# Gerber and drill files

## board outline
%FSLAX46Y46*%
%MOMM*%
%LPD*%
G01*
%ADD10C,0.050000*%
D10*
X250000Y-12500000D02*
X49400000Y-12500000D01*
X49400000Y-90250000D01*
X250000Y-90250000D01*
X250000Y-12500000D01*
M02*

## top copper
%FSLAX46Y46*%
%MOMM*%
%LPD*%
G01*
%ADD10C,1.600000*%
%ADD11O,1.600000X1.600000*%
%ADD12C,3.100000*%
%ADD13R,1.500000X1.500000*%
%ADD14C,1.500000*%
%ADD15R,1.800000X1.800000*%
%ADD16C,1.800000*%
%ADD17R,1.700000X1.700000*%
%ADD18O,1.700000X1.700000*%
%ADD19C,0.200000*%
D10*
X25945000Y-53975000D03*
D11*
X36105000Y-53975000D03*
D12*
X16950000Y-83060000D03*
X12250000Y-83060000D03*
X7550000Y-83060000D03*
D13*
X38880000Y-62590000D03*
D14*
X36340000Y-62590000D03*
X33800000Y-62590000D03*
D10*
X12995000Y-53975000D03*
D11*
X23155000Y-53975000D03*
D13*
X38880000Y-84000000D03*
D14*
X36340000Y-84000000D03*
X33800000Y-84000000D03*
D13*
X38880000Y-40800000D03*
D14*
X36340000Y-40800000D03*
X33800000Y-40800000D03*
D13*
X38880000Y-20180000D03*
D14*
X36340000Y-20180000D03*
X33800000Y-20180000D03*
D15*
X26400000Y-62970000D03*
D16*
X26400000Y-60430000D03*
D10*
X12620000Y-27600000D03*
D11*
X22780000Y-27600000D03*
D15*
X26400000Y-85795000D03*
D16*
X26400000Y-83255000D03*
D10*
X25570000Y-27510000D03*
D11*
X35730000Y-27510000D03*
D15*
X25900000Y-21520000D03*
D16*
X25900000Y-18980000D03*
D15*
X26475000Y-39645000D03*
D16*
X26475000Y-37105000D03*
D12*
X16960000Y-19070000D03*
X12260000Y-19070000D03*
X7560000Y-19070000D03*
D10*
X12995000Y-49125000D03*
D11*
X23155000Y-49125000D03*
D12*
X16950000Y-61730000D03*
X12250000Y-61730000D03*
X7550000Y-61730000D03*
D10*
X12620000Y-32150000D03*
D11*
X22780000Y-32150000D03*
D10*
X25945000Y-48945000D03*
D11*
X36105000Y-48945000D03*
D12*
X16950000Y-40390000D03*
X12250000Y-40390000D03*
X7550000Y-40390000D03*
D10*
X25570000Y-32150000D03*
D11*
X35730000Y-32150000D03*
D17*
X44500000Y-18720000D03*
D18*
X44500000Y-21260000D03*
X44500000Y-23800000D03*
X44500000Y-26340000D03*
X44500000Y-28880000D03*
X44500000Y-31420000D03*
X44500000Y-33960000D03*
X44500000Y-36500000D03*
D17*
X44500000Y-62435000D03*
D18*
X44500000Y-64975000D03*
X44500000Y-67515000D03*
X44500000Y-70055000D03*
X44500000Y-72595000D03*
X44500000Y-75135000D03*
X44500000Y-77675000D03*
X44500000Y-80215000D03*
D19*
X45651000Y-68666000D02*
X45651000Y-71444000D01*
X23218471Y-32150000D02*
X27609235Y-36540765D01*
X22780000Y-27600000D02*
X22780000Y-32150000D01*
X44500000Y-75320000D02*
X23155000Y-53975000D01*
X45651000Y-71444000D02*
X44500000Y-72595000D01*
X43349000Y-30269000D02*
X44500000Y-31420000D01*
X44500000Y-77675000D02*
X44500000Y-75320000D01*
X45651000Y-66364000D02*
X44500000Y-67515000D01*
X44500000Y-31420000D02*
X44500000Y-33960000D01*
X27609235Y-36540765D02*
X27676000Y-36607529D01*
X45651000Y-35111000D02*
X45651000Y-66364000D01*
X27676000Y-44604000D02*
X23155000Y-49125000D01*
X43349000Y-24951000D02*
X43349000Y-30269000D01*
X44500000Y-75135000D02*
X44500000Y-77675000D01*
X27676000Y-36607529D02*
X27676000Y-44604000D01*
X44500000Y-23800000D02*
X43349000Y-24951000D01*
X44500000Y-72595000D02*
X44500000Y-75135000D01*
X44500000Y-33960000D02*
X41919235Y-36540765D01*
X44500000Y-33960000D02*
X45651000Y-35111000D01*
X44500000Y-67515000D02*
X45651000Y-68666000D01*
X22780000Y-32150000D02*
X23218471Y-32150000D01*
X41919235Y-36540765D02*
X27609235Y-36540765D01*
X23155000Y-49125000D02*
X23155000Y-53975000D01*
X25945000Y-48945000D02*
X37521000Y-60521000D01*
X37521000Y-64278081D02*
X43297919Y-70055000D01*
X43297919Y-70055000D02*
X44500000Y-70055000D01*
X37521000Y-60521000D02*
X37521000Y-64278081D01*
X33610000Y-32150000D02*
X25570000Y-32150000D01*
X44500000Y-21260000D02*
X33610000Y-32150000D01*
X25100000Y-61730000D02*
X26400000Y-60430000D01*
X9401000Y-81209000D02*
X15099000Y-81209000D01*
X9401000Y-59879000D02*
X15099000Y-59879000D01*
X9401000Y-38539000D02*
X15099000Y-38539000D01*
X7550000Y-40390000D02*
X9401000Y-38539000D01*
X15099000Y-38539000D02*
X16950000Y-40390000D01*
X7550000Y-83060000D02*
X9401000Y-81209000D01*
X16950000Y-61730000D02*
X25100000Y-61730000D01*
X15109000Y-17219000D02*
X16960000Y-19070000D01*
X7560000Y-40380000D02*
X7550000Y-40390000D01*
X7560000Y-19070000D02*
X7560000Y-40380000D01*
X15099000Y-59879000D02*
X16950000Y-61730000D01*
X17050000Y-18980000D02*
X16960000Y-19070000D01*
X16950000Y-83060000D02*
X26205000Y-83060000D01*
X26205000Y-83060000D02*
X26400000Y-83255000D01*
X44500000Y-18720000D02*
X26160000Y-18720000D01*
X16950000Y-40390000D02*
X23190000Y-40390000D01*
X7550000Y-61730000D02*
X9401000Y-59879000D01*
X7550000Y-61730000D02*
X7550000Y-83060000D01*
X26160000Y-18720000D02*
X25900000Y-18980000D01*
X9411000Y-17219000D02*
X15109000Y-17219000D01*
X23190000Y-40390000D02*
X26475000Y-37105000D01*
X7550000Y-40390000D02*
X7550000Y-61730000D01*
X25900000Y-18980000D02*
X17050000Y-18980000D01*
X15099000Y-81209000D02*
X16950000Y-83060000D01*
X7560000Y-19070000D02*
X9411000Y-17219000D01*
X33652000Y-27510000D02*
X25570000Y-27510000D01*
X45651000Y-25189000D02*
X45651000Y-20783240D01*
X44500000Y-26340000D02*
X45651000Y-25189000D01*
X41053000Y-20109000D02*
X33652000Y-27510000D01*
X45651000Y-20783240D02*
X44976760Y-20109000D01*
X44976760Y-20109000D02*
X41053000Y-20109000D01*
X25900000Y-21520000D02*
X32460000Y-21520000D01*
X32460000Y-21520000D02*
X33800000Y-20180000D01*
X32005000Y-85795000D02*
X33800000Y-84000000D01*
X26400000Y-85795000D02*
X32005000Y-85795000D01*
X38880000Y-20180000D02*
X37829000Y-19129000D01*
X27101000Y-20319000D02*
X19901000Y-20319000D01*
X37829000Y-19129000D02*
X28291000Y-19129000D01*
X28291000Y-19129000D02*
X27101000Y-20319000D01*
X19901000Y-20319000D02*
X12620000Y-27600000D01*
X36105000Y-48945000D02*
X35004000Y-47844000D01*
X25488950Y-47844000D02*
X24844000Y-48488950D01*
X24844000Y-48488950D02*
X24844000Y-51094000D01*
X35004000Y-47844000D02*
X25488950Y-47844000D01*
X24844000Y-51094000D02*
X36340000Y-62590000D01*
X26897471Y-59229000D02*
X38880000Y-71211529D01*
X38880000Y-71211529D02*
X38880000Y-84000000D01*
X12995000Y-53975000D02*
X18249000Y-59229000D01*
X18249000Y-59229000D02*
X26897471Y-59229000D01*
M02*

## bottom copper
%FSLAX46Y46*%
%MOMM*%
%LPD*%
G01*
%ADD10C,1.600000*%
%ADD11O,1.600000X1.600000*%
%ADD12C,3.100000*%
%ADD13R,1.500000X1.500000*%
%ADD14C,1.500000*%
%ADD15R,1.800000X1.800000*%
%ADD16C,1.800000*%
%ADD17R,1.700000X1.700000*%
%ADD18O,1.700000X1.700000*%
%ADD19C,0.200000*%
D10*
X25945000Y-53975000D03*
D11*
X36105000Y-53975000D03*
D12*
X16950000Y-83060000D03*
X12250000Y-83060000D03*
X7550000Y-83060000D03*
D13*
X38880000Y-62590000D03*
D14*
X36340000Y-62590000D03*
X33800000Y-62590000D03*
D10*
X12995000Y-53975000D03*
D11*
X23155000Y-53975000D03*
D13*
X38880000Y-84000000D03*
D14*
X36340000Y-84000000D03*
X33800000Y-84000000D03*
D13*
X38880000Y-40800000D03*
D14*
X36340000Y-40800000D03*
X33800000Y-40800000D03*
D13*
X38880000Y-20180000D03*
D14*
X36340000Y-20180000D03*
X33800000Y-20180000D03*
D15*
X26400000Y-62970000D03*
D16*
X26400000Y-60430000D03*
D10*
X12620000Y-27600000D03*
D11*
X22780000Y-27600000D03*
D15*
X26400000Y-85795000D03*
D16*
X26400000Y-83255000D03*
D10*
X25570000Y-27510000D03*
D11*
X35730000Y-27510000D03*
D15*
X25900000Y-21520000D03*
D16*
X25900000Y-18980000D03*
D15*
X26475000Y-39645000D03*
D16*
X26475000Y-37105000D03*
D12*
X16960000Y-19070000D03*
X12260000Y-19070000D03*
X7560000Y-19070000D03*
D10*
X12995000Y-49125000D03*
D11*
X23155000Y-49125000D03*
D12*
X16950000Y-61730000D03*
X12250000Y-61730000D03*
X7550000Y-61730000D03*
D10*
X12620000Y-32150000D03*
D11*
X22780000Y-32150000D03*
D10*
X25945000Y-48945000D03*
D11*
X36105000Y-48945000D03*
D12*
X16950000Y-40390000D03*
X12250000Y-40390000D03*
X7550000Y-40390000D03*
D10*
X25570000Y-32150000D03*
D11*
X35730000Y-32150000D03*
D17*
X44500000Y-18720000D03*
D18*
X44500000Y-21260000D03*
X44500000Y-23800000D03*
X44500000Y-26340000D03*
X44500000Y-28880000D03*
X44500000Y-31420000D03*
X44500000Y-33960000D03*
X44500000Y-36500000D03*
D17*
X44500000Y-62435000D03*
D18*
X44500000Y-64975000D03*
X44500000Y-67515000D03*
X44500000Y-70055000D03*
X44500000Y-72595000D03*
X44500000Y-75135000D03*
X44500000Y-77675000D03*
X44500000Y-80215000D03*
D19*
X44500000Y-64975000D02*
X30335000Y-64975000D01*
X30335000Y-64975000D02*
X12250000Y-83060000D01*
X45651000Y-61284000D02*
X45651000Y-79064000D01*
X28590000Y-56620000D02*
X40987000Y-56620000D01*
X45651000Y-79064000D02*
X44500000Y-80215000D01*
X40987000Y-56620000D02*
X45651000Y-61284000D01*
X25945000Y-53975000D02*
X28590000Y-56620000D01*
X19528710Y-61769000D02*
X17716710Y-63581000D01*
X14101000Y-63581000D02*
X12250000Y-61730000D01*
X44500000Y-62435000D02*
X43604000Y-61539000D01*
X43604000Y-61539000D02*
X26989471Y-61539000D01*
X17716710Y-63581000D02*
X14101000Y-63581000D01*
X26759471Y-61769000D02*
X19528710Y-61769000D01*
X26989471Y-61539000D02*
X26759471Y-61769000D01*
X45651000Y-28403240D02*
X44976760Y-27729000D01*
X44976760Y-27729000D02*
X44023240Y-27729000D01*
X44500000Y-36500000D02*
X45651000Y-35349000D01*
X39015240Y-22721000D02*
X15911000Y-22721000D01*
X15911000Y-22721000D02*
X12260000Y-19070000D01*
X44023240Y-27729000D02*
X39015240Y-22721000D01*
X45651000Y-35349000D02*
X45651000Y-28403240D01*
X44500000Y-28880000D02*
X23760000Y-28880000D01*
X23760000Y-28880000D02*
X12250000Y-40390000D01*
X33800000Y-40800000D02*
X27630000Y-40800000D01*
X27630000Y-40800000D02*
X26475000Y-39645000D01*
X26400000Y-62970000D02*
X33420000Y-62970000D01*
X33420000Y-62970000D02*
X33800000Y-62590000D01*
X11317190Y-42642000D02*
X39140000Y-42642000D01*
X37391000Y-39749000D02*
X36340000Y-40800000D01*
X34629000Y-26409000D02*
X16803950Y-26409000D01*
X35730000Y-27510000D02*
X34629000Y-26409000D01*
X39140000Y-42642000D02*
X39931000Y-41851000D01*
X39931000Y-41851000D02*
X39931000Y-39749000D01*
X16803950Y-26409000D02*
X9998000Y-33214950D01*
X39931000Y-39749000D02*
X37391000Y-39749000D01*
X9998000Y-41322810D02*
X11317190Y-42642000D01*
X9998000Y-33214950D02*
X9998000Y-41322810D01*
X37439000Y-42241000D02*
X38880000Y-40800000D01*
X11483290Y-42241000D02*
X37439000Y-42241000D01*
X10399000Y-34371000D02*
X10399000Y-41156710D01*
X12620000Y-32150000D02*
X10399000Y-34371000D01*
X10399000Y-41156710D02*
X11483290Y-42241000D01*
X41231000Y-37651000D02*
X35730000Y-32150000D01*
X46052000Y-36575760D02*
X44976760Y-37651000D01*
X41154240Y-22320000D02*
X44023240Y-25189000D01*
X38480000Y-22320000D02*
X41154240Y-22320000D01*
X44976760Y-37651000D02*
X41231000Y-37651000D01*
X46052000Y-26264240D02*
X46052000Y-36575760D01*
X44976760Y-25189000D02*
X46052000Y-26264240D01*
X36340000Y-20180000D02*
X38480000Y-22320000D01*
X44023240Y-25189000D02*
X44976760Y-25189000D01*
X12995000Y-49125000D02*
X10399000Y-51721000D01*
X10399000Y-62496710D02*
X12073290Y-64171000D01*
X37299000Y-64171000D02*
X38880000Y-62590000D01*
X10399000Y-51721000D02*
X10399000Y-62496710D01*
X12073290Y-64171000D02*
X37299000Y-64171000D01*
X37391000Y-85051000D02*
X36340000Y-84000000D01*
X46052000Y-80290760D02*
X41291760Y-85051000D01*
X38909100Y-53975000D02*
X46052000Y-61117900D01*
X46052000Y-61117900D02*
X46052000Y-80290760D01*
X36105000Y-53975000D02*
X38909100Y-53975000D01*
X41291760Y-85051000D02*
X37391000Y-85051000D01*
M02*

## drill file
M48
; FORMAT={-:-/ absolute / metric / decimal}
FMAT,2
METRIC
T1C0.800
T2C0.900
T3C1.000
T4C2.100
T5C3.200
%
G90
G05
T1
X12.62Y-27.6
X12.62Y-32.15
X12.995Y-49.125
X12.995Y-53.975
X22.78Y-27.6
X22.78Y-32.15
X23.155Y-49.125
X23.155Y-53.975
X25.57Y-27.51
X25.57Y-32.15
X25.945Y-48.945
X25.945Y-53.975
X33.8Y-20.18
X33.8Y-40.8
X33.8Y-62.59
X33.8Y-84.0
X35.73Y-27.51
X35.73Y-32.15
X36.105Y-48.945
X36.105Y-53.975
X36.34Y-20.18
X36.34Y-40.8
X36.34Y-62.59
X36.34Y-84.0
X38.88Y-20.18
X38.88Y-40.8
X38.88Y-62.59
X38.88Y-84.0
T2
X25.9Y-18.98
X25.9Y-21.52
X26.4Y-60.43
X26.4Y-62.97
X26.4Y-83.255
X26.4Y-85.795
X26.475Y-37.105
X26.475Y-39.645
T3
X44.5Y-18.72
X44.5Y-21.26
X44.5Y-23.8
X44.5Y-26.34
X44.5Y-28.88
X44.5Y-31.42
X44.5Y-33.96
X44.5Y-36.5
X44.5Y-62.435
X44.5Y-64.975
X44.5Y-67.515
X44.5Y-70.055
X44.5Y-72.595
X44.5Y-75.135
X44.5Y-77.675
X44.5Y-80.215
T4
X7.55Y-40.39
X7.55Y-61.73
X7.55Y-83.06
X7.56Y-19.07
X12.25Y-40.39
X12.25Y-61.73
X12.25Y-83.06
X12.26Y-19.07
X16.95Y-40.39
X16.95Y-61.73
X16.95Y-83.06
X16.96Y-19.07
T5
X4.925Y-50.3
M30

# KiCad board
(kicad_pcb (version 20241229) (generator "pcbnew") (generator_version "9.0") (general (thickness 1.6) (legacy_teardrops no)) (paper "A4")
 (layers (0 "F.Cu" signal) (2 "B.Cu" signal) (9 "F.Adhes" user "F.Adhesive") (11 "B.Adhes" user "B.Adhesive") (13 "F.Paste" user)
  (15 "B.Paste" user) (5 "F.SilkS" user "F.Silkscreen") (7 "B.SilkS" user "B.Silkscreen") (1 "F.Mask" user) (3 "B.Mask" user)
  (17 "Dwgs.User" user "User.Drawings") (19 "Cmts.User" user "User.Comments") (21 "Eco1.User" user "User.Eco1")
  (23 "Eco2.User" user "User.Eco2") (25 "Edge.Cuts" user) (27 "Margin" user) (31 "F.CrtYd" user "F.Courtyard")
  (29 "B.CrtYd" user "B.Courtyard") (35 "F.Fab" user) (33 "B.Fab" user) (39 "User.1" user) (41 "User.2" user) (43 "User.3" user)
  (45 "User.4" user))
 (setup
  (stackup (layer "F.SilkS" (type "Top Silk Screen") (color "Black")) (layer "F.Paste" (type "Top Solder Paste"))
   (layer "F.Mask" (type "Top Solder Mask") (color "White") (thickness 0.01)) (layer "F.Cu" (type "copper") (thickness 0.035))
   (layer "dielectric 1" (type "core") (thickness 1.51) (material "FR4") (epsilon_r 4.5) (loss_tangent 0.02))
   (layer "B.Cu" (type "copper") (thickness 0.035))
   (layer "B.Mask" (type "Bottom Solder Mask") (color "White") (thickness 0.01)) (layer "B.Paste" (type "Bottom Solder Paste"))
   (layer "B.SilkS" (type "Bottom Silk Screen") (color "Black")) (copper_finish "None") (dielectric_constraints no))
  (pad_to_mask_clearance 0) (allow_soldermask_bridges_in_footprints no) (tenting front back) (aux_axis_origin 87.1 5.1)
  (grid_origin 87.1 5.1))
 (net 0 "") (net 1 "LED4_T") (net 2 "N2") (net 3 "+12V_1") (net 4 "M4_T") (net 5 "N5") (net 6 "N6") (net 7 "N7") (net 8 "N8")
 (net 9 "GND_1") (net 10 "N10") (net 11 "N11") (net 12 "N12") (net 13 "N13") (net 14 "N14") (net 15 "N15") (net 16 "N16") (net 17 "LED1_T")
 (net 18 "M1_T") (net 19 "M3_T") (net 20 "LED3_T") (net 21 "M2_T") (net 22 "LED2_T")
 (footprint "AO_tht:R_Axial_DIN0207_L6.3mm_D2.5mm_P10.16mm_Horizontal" (layer "F.Cu") (at 25.945 53.975)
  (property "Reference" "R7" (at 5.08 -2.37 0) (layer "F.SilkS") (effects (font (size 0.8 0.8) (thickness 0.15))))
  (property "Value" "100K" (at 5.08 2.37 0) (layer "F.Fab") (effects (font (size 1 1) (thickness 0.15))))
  (pad "1" thru_hole circle (at 0 0) (size 1.6 1.6) (drill 0.8) (layers "*.Cu" "*.Mask") (remove_unused_layers no) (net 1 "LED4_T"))
  (pad "2" thru_hole oval (at 10.16 0) (size 1.6 1.6) (drill 0.8) (layers "*.Cu" "*.Mask") (remove_unused_layers no) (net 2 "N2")))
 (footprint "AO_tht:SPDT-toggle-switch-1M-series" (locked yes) (layer "F.Cu") (at 12.25 83.06 90)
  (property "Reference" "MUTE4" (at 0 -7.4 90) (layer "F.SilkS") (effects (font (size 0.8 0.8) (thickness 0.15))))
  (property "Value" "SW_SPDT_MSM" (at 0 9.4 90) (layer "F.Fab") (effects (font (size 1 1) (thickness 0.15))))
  (pad "1" thru_hole circle (at 0 4.7 90) (size 3.1 3.1) (drill 2.1) (layers "*.Cu" "*.Mask") (remove_unused_layers no) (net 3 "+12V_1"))
  (pad "2" thru_hole circle (at 0 0 90) (size 3.1 3.1) (drill 2.1) (layers "*.Cu" "*.Mask") (remove_unused_layers no) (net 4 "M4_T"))
  (pad "3" thru_hole circle (at 0 -4.7 90) (size 3.1 3.1) (drill 2.1) (layers "*.Cu" "*.Mask") (remove_unused_layers no) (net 3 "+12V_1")))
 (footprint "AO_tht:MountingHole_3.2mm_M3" (layer "F.Cu") (at 4.925 50.3)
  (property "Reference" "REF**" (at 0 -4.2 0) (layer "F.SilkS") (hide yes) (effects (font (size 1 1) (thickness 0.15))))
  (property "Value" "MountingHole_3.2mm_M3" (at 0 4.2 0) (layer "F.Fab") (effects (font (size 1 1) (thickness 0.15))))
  (pad "" np_thru_hole circle (at 0 0) (size 3.2 3.2) (drill 3.2) (layers "*.Cu" "*.Mask")))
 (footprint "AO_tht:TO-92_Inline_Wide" (layer "F.Cu") (at 38.88 62.59 180)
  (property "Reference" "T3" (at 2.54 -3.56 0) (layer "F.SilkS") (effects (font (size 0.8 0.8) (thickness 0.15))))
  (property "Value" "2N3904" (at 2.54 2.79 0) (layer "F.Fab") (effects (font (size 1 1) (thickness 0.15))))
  (pad "1" thru_hole rect (at 0 0 270) (size 1.5 1.5) (drill 0.8) (layers "*.Cu" "*.Mask") (remove_unused_layers no) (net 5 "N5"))
  (pad "2" thru_hole circle (at 2.54 0 270) (size 1.5 1.5) (drill 0.8) (layers "*.Cu" "*.Mask") (remove_unused_layers no) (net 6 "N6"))
  (pad "3" thru_hole circle (at 5.08 0 270) (size 1.5 1.5) (drill 0.8) (layers "*.Cu" "*.Mask") (remove_unused_layers no) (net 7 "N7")))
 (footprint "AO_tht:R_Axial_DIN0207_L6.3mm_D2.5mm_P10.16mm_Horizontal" (layer "F.Cu") (at 12.995 53.975)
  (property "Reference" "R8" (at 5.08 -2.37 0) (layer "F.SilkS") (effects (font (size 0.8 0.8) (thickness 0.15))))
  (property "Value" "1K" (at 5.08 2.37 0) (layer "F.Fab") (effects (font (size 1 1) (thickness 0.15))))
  (pad "1" thru_hole circle (at 0 0) (size 1.6 1.6) (drill 0.8) (layers "*.Cu" "*.Mask") (remove_unused_layers no) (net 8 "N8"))
  (pad "2" thru_hole oval (at 10.16 0) (size 1.6 1.6) (drill 0.8) (layers "*.Cu" "*.Mask") (remove_unused_layers no) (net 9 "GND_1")))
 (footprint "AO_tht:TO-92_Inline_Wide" (layer "F.Cu") (at 38.88 84 180)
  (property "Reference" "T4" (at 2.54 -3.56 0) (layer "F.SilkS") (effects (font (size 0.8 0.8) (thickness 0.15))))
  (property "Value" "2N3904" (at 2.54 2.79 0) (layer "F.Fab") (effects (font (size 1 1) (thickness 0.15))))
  (pad "1" thru_hole rect (at 0 0 270) (size 1.5 1.5) (drill 0.8) (layers "*.Cu" "*.Mask") (remove_unused_layers no) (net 8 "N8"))
  (pad "2" thru_hole circle (at 2.54 0 270) (size 1.5 1.5) (drill 0.8) (layers "*.Cu" "*.Mask") (remove_unused_layers no) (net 2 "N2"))
  (pad "3" thru_hole circle (at 5.08 0 270) (size 1.5 1.5) (drill 0.8) (layers "*.Cu" "*.Mask") (remove_unused_layers no) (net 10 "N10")))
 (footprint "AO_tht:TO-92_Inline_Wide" (layer "F.Cu") (at 38.88 40.8 180)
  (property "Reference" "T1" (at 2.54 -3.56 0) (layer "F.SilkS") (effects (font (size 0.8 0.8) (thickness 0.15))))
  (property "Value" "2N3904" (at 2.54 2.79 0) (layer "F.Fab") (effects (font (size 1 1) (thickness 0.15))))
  (pad "1" thru_hole rect (at 0 0 270) (size 1.5 1.5) (drill 0.8) (layers "*.Cu" "*.Mask") (remove_unused_layers no) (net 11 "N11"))
  (pad "2" thru_hole circle (at 2.54 0 270) (size 1.5 1.5) (drill 0.8) (layers "*.Cu" "*.Mask") (remove_unused_layers no) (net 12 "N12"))
  (pad "3" thru_hole circle (at 5.08 0 270) (size 1.5 1.5) (drill 0.8) (layers "*.Cu" "*.Mask") (remove_unused_layers no) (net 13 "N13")))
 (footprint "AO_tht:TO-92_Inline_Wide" (layer "F.Cu") (at 38.88 20.18 180)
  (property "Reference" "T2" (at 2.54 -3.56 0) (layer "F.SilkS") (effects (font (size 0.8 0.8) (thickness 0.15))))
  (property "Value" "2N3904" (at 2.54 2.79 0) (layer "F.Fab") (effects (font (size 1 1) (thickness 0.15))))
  (pad "1" thru_hole rect (at 0 0 270) (size 1.5 1.5) (drill 0.8) (layers "*.Cu" "*.Mask") (remove_unused_layers no) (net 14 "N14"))
  (pad "2" thru_hole circle (at 2.54 0 270) (size 1.5 1.5) (drill 0.8) (layers "*.Cu" "*.Mask") (remove_unused_layers no) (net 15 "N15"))
  (pad "3" thru_hole circle (at 5.08 0 270) (size 1.5 1.5) (drill 0.8) (layers "*.Cu" "*.Mask") (remove_unused_layers no) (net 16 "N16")))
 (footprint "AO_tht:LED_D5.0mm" (layer "F.Cu") (at 26.4 62.97 90)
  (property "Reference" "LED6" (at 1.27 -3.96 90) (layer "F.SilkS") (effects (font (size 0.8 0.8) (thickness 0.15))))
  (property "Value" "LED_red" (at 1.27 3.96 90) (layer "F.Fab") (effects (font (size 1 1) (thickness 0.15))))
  (pad "1" thru_hole rect (at 0 0 90) (size 1.8 1.8) (drill 0.9) (layers "*.Cu" "*.Mask") (remove_unused_layers no) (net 7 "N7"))
  (pad "2" thru_hole circle (at 2.54 0 90) (size 1.8 1.8) (drill 0.9) (layers "*.Cu" "*.Mask") (remove_unused_layers no) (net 3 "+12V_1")))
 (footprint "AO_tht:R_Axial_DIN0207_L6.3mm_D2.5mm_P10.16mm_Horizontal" (layer "F.Cu") (at 12.62 27.6)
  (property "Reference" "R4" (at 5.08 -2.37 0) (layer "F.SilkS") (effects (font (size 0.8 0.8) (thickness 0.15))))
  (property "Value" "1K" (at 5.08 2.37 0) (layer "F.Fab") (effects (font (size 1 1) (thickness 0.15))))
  (pad "1" thru_hole circle (at 0 0) (size 1.6 1.6) (drill 0.8) (layers "*.Cu" "*.Mask") (remove_unused_layers no) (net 14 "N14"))
  (pad "2" thru_hole oval (at 10.16 0) (size 1.6 1.6) (drill 0.8) (layers "*.Cu" "*.Mask") (remove_unused_layers no) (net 9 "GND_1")))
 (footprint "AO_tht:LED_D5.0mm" (layer "F.Cu") (at 26.4 85.795 90)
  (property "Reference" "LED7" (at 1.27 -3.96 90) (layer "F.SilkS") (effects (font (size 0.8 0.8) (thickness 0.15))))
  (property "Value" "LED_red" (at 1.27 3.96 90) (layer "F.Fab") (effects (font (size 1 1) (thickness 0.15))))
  (pad "1" thru_hole rect (at 0 0 90) (size 1.8 1.8) (drill 0.9) (layers "*.Cu" "*.Mask") (remove_unused_layers no) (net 10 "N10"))
  (pad "2" thru_hole circle (at 2.54 0 90) (size 1.8 1.8) (drill 0.9) (layers "*.Cu" "*.Mask") (remove_unused_layers no) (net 3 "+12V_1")))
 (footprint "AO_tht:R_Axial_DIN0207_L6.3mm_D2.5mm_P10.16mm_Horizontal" (layer "F.Cu") (at 25.57 27.51)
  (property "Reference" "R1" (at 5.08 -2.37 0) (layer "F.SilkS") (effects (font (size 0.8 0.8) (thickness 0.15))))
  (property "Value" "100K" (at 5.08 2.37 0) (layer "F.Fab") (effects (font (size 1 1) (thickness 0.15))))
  (pad "1" thru_hole circle (at 0 0) (size 1.6 1.6) (drill 0.8) (layers "*.Cu" "*.Mask") (remove_unused_layers no) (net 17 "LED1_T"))
  (pad "2" thru_hole oval (at 10.16 0) (size 1.6 1.6) (drill 0.8) (layers "*.Cu" "*.Mask") (remove_unused_layers no) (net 12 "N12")))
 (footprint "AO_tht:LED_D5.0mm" (layer "F.Cu") (at 25.9 21.52 90)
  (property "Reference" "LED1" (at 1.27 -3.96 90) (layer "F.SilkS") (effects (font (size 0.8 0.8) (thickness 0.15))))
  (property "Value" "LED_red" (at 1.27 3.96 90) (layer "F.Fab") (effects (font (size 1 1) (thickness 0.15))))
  (pad "1" thru_hole rect (at 0 0 90) (size 1.8 1.8) (drill 0.9) (layers "*.Cu" "*.Mask") (remove_unused_layers no) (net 16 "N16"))
  (pad "2" thru_hole circle (at 2.54 0 90) (size 1.8 1.8) (drill 0.9) (layers "*.Cu" "*.Mask") (remove_unused_layers no) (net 3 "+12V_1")))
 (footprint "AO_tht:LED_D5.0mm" (layer "F.Cu") (at 26.475 39.645 90)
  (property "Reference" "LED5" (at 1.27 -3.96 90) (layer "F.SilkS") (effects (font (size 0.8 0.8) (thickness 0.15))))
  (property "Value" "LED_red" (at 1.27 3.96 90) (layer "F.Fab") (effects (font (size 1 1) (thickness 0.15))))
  (pad "1" thru_hole rect (at 0 0 90) (size 1.8 1.8) (drill 0.9) (layers "*.Cu" "*.Mask") (remove_unused_layers no) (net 13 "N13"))
  (pad "2" thru_hole circle (at 2.54 0 90) (size 1.8 1.8) (drill 0.9) (layers "*.Cu" "*.Mask") (remove_unused_layers no) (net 3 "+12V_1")))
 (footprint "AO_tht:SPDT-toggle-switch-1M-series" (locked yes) (layer "F.Cu") (at 12.26 19.07 90)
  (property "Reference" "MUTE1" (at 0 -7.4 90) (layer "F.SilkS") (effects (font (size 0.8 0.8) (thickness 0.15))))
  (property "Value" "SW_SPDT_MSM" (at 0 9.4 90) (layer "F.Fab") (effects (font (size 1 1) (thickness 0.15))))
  (pad "1" thru_hole circle (at 0 4.7 90) (size 3.1 3.1) (drill 2.1) (layers "*.Cu" "*.Mask") (remove_unused_layers no) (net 3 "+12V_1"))
  (pad "2" thru_hole circle (at 0 0 90) (size 3.1 3.1) (drill 2.1) (layers "*.Cu" "*.Mask") (remove_unused_layers no) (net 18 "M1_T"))
  (pad "3" thru_hole circle (at 0 -4.7 90) (size 3.1 3.1) (drill 2.1) (layers "*.Cu" "*.Mask") (remove_unused_layers no) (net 3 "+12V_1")))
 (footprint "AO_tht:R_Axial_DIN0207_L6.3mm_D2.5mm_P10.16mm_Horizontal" (layer "F.Cu") (at 12.995 49.125)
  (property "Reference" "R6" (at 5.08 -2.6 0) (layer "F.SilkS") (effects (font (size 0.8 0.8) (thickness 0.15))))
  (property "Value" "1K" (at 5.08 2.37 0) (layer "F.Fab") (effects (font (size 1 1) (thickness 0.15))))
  (pad "1" thru_hole circle (at 0 0) (size 1.6 1.6) (drill 0.8) (layers "*.Cu" "*.Mask") (remove_unused_layers no) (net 5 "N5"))
  (pad "2" thru_hole oval (at 10.16 0) (size 1.6 1.6) (drill 0.8) (layers "*.Cu" "*.Mask") (remove_unused_layers no) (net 9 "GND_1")))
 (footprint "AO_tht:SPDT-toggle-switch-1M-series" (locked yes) (layer "F.Cu") (at 12.25 61.73 90)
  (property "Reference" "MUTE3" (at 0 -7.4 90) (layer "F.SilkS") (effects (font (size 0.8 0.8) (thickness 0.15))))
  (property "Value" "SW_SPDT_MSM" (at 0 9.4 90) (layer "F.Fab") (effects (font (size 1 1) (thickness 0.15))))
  (pad "1" thru_hole circle (at 0 4.7 90) (size 3.1 3.1) (drill 2.1) (layers "*.Cu" "*.Mask") (remove_unused_layers no) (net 3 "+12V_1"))
  (pad "2" thru_hole circle (at 0 0 90) (size 3.1 3.1) (drill 2.1) (layers "*.Cu" "*.Mask") (remove_unused_layers no) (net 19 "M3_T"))
  (pad "3" thru_hole circle (at 0 -4.7 90) (size 3.1 3.1) (drill 2.1) (layers "*.Cu" "*.Mask") (remove_unused_layers no) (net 3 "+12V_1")))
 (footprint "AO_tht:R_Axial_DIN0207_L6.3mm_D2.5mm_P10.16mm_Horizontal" (layer "F.Cu") (at 12.62 32.15)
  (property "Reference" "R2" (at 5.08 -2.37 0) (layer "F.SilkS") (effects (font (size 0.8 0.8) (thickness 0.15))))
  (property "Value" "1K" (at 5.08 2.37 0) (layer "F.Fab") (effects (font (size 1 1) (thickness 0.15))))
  (pad "1" thru_hole circle (at 0 0) (size 1.6 1.6) (drill 0.8) (layers "*.Cu" "*.Mask") (remove_unused_layers no) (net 11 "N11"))
  (pad "2" thru_hole oval (at 10.16 0) (size 1.6 1.6) (drill 0.8) (layers "*.Cu" "*.Mask") (remove_unused_layers no) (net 9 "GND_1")))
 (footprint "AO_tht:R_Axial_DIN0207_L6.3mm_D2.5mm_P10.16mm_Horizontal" (layer "F.Cu") (at 25.945 48.945)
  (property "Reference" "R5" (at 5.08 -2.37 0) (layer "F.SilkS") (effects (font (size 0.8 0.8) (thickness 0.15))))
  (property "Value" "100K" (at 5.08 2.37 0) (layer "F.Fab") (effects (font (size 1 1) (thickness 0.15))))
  (pad "1" thru_hole circle (at 0 0) (size 1.6 1.6) (drill 0.8) (layers "*.Cu" "*.Mask") (remove_unused_layers no) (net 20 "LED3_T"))
  (pad "2" thru_hole oval (at 10.16 0) (size 1.6 1.6) (drill 0.8) (layers "*.Cu" "*.Mask") (remove_unused_layers no) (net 6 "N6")))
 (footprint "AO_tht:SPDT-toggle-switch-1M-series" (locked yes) (layer "F.Cu") (at 12.25 40.39 90)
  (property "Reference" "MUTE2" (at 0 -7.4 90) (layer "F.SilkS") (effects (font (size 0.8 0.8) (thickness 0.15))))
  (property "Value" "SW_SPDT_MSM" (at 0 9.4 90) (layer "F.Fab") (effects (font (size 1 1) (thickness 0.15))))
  (pad "1" thru_hole circle (at 0 4.7 90) (size 3.1 3.1) (drill 2.1) (layers "*.Cu" "*.Mask") (remove_unused_layers no) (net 3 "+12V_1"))
  (pad "2" thru_hole circle (at 0 0 90) (size 3.1 3.1) (drill 2.1) (layers "*.Cu" "*.Mask") (remove_unused_layers no) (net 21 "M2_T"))
  (pad "3" thru_hole circle (at 0 -4.7 90) (size 3.1 3.1) (drill 2.1) (layers "*.Cu" "*.Mask") (remove_unused_layers no) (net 3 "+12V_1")))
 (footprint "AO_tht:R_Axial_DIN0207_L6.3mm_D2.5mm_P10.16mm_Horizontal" (layer "F.Cu") (at 25.57 32.15)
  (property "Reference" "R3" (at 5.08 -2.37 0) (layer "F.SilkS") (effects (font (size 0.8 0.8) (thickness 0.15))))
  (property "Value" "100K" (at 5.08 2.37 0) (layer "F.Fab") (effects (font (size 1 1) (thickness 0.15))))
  (pad "1" thru_hole circle (at 0 0) (size 1.6 1.6) (drill 0.8) (layers "*.Cu" "*.Mask") (remove_unused_layers no) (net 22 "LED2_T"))
  (pad "2" thru_hole oval (at 10.16 0) (size 1.6 1.6) (drill 0.8) (layers "*.Cu" "*.Mask") (remove_unused_layers no) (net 15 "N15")))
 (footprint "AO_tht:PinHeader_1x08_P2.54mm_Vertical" (layer "B.Cu") (at 44.373 27.61 -90)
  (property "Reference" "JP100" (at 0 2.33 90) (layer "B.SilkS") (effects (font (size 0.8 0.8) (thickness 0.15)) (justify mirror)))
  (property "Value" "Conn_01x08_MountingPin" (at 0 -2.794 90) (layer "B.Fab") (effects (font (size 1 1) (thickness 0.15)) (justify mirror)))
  (pad "1" thru_hole rect (at -8.89 -0.127 180) (size 1.7 1.7) (drill 1) (layers "*.Cu" "*.Mask") (remove_unused_layers no) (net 3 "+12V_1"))
  (pad "2" thru_hole oval (at -6.35 -0.127 180) (size 1.7 1.7) (drill 1) (layers "*.Cu" "*.Mask") (remove_unused_layers no)
   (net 22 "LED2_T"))
  (pad "3" thru_hole oval (at -3.81 -0.127 180) (size 1.7 1.7) (drill 1) (layers "*.Cu" "*.Mask") (remove_unused_layers no) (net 9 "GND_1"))
  (pad "4" thru_hole oval (at -1.27 -0.127 180) (size 1.7 1.7) (drill 1) (layers "*.Cu" "*.Mask") (remove_unused_layers no)
   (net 17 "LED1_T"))
  (pad "5" thru_hole oval (at 1.27 -0.127 180) (size 1.7 1.7) (drill 1) (layers "*.Cu" "*.Mask") (remove_unused_layers no) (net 21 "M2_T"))
  (pad "6" thru_hole oval (at 3.81 -0.127 180) (size 1.7 1.7) (drill 1) (layers "*.Cu" "*.Mask") (remove_unused_layers no) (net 9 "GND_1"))
  (pad "7" thru_hole oval (at 6.35 -0.127 180) (size 1.7 1.7) (drill 1) (layers "*.Cu" "*.Mask") (remove_unused_layers no) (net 9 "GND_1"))
  (pad "8" thru_hole oval (at 8.89 -0.127 180) (size 1.7 1.7) (drill 1) (layers "*.Cu" "*.Mask") (remove_unused_layers no) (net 18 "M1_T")))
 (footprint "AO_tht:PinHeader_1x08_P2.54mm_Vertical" (layer "B.Cu") (at 44.373 71.325 -90)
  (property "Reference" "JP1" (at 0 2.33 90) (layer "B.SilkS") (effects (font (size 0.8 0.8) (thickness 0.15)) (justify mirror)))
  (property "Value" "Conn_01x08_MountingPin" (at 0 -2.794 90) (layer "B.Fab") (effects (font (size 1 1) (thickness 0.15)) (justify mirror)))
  (pad "1" thru_hole rect (at -8.89 -0.127 180) (size 1.7 1.7) (drill 1) (layers "*.Cu" "*.Mask") (remove_unused_layers no) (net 19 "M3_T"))
  (pad "2" thru_hole oval (at -6.35 -0.127 180) (size 1.7 1.7) (drill 1) (layers "*.Cu" "*.Mask") (remove_unused_layers no) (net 4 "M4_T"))
  (pad "3" thru_hole oval (at -3.81 -0.127 180) (size 1.7 1.7) (drill 1) (layers "*.Cu" "*.Mask") (remove_unused_layers no) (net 9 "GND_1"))
  (pad "4" thru_hole oval (at -1.27 -0.127 180) (size 1.7 1.7) (drill 1) (layers "*.Cu" "*.Mask") (remove_unused_layers no)
   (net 20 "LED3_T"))
  (pad "5" thru_hole oval (at 1.27 -0.127 180) (size 1.7 1.7) (drill 1) (layers "*.Cu" "*.Mask") (remove_unused_layers no) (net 9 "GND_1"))
  (pad "6" thru_hole oval (at 3.81 -0.127 180) (size 1.7 1.7) (drill 1) (layers "*.Cu" "*.Mask") (remove_unused_layers no) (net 9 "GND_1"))
  (pad "7" thru_hole oval (at 6.35 -0.127 180) (size 1.7 1.7) (drill 1) (layers "*.Cu" "*.Mask") (remove_unused_layers no) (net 9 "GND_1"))
  (pad "8" thru_hole oval (at 8.89 -0.127 180) (size 1.7 1.7) (drill 1) (layers "*.Cu" "*.Mask") (remove_unused_layers no) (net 1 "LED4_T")))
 (gr_rect (start 0.25 12.5) (end 49.4 90.25) (stroke (width 0.05) (type solid)) (fill no) (layer "Edge.Cuts"))
 (segment (start 45.651 68.666) (end 45.651 71.444) (width 0.2) (layer "F.Cu") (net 9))
 (segment (start 23.218471 32.15) (end 27.609235 36.540765) (width 0.2) (layer "F.Cu") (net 9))
 (segment (start 22.78 27.6) (end 22.78 32.15) (width 0.2) (layer "F.Cu") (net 9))
 (segment (start 44.5 75.32) (end 23.155 53.975) (width 0.2) (layer "F.Cu") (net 9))
 (segment (start 45.651 71.444) (end 44.5 72.595) (width 0.2) (layer "F.Cu") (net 9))
 (segment (start 43.349 30.269) (end 44.5 31.42) (width 0.2) (layer "F.Cu") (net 9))
 (segment (start 44.5 77.675) (end 44.5 75.32) (width 0.2) (layer "F.Cu") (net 9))
 (segment (start 45.651 66.364) (end 44.5 67.515) (width 0.2) (layer "F.Cu") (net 9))
 (segment (start 44.5 31.42) (end 44.5 33.96) (width 0.2) (layer "F.Cu") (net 9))
 (segment (start 27.609235 36.540765) (end 27.676 36.607529) (width 0.2) (layer "F.Cu") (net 9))
 (segment (start 45.651 35.111) (end 45.651 66.364) (width 0.2) (layer "F.Cu") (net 9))
 (segment (start 27.676 44.604) (end 23.155 49.125) (width 0.2) (layer "F.Cu") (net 9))
 (segment (start 43.349 24.951) (end 43.349 30.269) (width 0.2) (layer "F.Cu") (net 9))
 (segment (start 44.5 75.135) (end 44.5 77.675) (width 0.2) (layer "F.Cu") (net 9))
 (segment (start 27.676 36.607529) (end 27.676 44.604) (width 0.2) (layer "F.Cu") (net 9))
 (segment (start 44.5 23.8) (end 43.349 24.951) (width 0.2) (layer "F.Cu") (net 9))
 (segment (start 44.5 72.595) (end 44.5 75.135) (width 0.2) (layer "F.Cu") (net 9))
 (segment (start 44.5 33.96) (end 41.919235 36.540765) (width 0.2) (layer "F.Cu") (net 9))
 (segment (start 44.5 33.96) (end 45.651 35.111) (width 0.2) (layer "F.Cu") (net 9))
 (segment (start 44.5 67.515) (end 45.651 68.666) (width 0.2) (layer "F.Cu") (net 9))
 (segment (start 22.78 32.15) (end 23.218471 32.15) (width 0.2) (layer "F.Cu") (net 9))
 (segment (start 41.919235 36.540765) (end 27.609235 36.540765) (width 0.2) (layer "F.Cu") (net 9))
 (segment (start 23.155 49.125) (end 23.155 53.975) (width 0.2) (layer "F.Cu") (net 9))
 (segment (start 25.945 48.945) (end 37.521 60.521) (width 0.2) (layer "F.Cu") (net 20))
 (segment (start 37.521 64.278081) (end 43.297919 70.055) (width 0.2) (layer "F.Cu") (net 20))
 (segment (start 43.297919 70.055) (end 44.5 70.055) (width 0.2) (layer "F.Cu") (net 20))
 (segment (start 37.521 60.521) (end 37.521 64.278081) (width 0.2) (layer "F.Cu") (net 20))
 (segment (start 44.5 64.975) (end 30.335 64.975) (width 0.2) (layer "B.Cu") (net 4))
 (segment (start 30.335 64.975) (end 12.25 83.06) (width 0.2) (layer "B.Cu") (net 4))
 (segment (start 45.651 61.284) (end 45.651 79.064) (width 0.2) (layer "B.Cu") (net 1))
 (segment (start 28.59 56.62) (end 40.987 56.62) (width 0.2) (layer "B.Cu") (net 1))
 (segment (start 45.651 79.064) (end 44.5 80.215) (width 0.2) (layer "B.Cu") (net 1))
 (segment (start 40.987 56.62) (end 45.651 61.284) (width 0.2) (layer "B.Cu") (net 1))
 (segment (start 25.945 53.975) (end 28.59 56.62) (width 0.2) (layer "B.Cu") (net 1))
 (segment (start 19.52871 61.769) (end 17.71671 63.581) (width 0.2) (layer "B.Cu") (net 19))
 (segment (start 14.101 63.581) (end 12.25 61.73) (width 0.2) (layer "B.Cu") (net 19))
 (segment (start 44.5 62.435) (end 43.604 61.539) (width 0.2) (layer "B.Cu") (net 19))
 (segment (start 43.604 61.539) (end 26.989471 61.539) (width 0.2) (layer "B.Cu") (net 19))
 (segment (start 17.71671 63.581) (end 14.101 63.581) (width 0.2) (layer "B.Cu") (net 19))
 (segment (start 26.759471 61.769) (end 19.52871 61.769) (width 0.2) (layer "B.Cu") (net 19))
 (segment (start 26.989471 61.539) (end 26.759471 61.769) (width 0.2) (layer "B.Cu") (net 19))
 (segment (start 45.651 28.40324) (end 44.97676 27.729) (width 0.2) (layer "B.Cu") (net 18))
 (segment (start 44.97676 27.729) (end 44.02324 27.729) (width 0.2) (layer "B.Cu") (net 18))
 (segment (start 44.5 36.5) (end 45.651 35.349) (width 0.2) (layer "B.Cu") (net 18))
 (segment (start 39.01524 22.721) (end 15.911 22.721) (width 0.2) (layer "B.Cu") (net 18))
 (segment (start 15.911 22.721) (end 12.26 19.07) (width 0.2) (layer "B.Cu") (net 18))
 (segment (start 44.02324 27.729) (end 39.01524 22.721) (width 0.2) (layer "B.Cu") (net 18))
 (segment (start 45.651 35.349) (end 45.651 28.40324) (width 0.2) (layer "B.Cu") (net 18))
 (segment (start 33.61 32.15) (end 25.57 32.15) (width 0.2) (layer "F.Cu") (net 22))
 (segment (start 44.5 21.26) (end 33.61 32.15) (width 0.2) (layer "F.Cu") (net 22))
 (segment (start 25.1 61.73) (end 26.4 60.43) (width 0.2) (layer "F.Cu") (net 3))
 (segment (start 9.401 81.209) (end 15.099 81.209) (width 0.2) (layer "F.Cu") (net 3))
 (segment (start 9.401 59.879) (end 15.099 59.879) (width 0.2) (layer "F.Cu") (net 3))
 (segment (start 9.401 38.539) (end 15.099 38.539) (width 0.2) (layer "F.Cu") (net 3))
 (segment (start 7.55 40.39) (end 9.401 38.539) (width 0.2) (layer "F.Cu") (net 3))
 (segment (start 15.099 38.539) (end 16.95 40.39) (width 0.2) (layer "F.Cu") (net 3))
 (segment (start 7.55 83.06) (end 9.401 81.209) (width 0.2) (layer "F.Cu") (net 3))
 (segment (start 16.95 61.73) (end 25.1 61.73) (width 0.2) (layer "F.Cu") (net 3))
 (segment (start 15.109 17.219) (end 16.96 19.07) (width 0.2) (layer "F.Cu") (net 3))
 (segment (start 7.56 40.38) (end 7.55 40.39) (width 0.2) (layer "F.Cu") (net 3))
 (segment (start 7.56 19.07) (end 7.56 40.38) (width 0.2) (layer "F.Cu") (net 3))
 (segment (start 15.099 59.879) (end 16.95 61.73) (width 0.2) (layer "F.Cu") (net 3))
 (segment (start 17.05 18.98) (end 16.96 19.07) (width 0.2) (layer "F.Cu") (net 3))
 (segment (start 16.95 83.06) (end 26.205 83.06) (width 0.2) (layer "F.Cu") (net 3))
 (segment (start 26.205 83.06) (end 26.4 83.255) (width 0.2) (layer "F.Cu") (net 3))
 (segment (start 44.5 18.72) (end 26.16 18.72) (width 0.2) (layer "F.Cu") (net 3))
 (segment (start 16.95 40.39) (end 23.19 40.39) (width 0.2) (layer "F.Cu") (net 3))
 (segment (start 7.55 61.73) (end 9.401 59.879) (width 0.2) (layer "F.Cu") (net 3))
 (segment (start 7.55 61.73) (end 7.55 83.06) (width 0.2) (layer "F.Cu") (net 3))
 (segment (start 26.16 18.72) (end 25.9 18.98) (width 0.2) (layer "F.Cu") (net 3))
 (segment (start 9.411 17.219) (end 15.109 17.219) (width 0.2) (layer "F.Cu") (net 3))
 (segment (start 23.19 40.39) (end 26.475 37.105) (width 0.2) (layer "F.Cu") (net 3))
 (segment (start 7.55 40.39) (end 7.55 61.73) (width 0.2) (layer "F.Cu") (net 3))
 (segment (start 25.9 18.98) (end 17.05 18.98) (width 0.2) (layer "F.Cu") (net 3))
 (segment (start 15.099 81.209) (end 16.95 83.06) (width 0.2) (layer "F.Cu") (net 3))
 (segment (start 7.56 19.07) (end 9.411 17.219) (width 0.2) (layer "F.Cu") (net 3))
 (segment (start 44.5 28.88) (end 23.76 28.88) (width 0.2) (layer "B.Cu") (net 21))
 (segment (start 23.76 28.88) (end 12.25 40.39) (width 0.2) (layer "B.Cu") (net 21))
 (segment (start 33.652 27.51) (end 25.57 27.51) (width 0.2) (layer "F.Cu") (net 17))
 (segment (start 45.651 25.189) (end 45.651 20.78324) (width 0.2) (layer "F.Cu") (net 17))
 (segment (start 44.5 26.34) (end 45.651 25.189) (width 0.2) (layer "F.Cu") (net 17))
 (segment (start 41.053 20.109) (end 33.652 27.51) (width 0.2) (layer "F.Cu") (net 17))
 (segment (start 45.651 20.78324) (end 44.97676 20.109) (width 0.2) (layer "F.Cu") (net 17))
 (segment (start 44.97676 20.109) (end 41.053 20.109) (width 0.2) (layer "F.Cu") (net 17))
 (segment (start 25.9 21.52) (end 32.46 21.52) (width 0.2) (layer "F.Cu") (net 16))
 (segment (start 32.46 21.52) (end 33.8 20.18) (width 0.2) (layer "F.Cu") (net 16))
 (segment (start 33.8 40.8) (end 27.63 40.8) (width 0.2) (layer "B.Cu") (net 13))
 (segment (start 27.63 40.8) (end 26.475 39.645) (width 0.2) (layer "B.Cu") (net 13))
 (segment (start 26.4 62.97) (end 33.42 62.97) (width 0.2) (layer "B.Cu") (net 7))
 (segment (start 33.42 62.97) (end 33.8 62.59) (width 0.2) (layer "B.Cu") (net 7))
 (segment (start 32.005 85.795) (end 33.8 84) (width 0.2) (layer "F.Cu") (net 10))
 (segment (start 26.4 85.795) (end 32.005 85.795) (width 0.2) (layer "F.Cu") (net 10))
 (segment (start 11.31719 42.642) (end 39.14 42.642) (width 0.2) (layer "B.Cu") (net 12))
 (segment (start 37.391 39.749) (end 36.34 40.8) (width 0.2) (layer "B.Cu") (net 12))
 (segment (start 34.629 26.409) (end 16.80395 26.409) (width 0.2) (layer "B.Cu") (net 12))
 (segment (start 35.73 27.51) (end 34.629 26.409) (width 0.2) (layer "B.Cu") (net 12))
 (segment (start 39.14 42.642) (end 39.931 41.851) (width 0.2) (layer "B.Cu") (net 12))
 (segment (start 39.931 41.851) (end 39.931 39.749) (width 0.2) (layer "B.Cu") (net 12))
 (segment (start 16.80395 26.409) (end 9.998 33.21495) (width 0.2) (layer "B.Cu") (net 12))
 (segment (start 39.931 39.749) (end 37.391 39.749) (width 0.2) (layer "B.Cu") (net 12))
 (segment (start 9.998 41.32281) (end 11.31719 42.642) (width 0.2) (layer "B.Cu") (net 12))
 (segment (start 9.998 33.21495) (end 9.998 41.32281) (width 0.2) (layer "B.Cu") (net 12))
 (segment (start 37.439 42.241) (end 38.88 40.8) (width 0.2) (layer "B.Cu") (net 11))
 (segment (start 11.48329 42.241) (end 37.439 42.241) (width 0.2) (layer "B.Cu") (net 11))
 (segment (start 10.399 34.371) (end 10.399 41.15671) (width 0.2) (layer "B.Cu") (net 11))
 (segment (start 12.62 32.15) (end 10.399 34.371) (width 0.2) (layer "B.Cu") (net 11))
 (segment (start 10.399 41.15671) (end 11.48329 42.241) (width 0.2) (layer "B.Cu") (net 11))
 (segment (start 41.231 37.651) (end 35.73 32.15) (width 0.2) (layer "B.Cu") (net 15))
 (segment (start 46.052 36.57576) (end 44.97676 37.651) (width 0.2) (layer "B.Cu") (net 15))
 (segment (start 41.15424 22.32) (end 44.02324 25.189) (width 0.2) (layer "B.Cu") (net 15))
 (segment (start 38.48 22.32) (end 41.15424 22.32) (width 0.2) (layer "B.Cu") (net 15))
 (segment (start 44.97676 37.651) (end 41.231 37.651) (width 0.2) (layer "B.Cu") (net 15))
 (segment (start 46.052 26.26424) (end 46.052 36.57576) (width 0.2) (layer "B.Cu") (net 15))
 (segment (start 44.97676 25.189) (end 46.052 26.26424) (width 0.2) (layer "B.Cu") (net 15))
 (segment (start 36.34 20.18) (end 38.48 22.32) (width 0.2) (layer "B.Cu") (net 15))
 (segment (start 44.02324 25.189) (end 44.97676 25.189) (width 0.2) (layer "B.Cu") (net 15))
 (segment (start 38.88 20.18) (end 37.829 19.129) (width 0.2) (layer "F.Cu") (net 14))
 (segment (start 27.101 20.319) (end 19.901 20.319) (width 0.2) (layer "F.Cu") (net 14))
 (segment (start 37.829 19.129) (end 28.291 19.129) (width 0.2) (layer "F.Cu") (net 14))
 (segment (start 28.291 19.129) (end 27.101 20.319) (width 0.2) (layer "F.Cu") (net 14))
 (segment (start 19.901 20.319) (end 12.62 27.6) (width 0.2) (layer "F.Cu") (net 14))
 (segment (start 36.105 48.945) (end 35.004 47.844) (width 0.2) (layer "F.Cu") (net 6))
 (segment (start 25.48895 47.844) (end 24.844 48.48895) (width 0.2) (layer "F.Cu") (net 6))
 (segment (start 24.844 48.48895) (end 24.844 51.094) (width 0.2) (layer "F.Cu") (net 6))
 (segment (start 35.004 47.844) (end 25.48895 47.844) (width 0.2) (layer "F.Cu") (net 6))
 (segment (start 24.844 51.094) (end 36.34 62.59) (width 0.2) (layer "F.Cu") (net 6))
 (segment (start 12.995 49.125) (end 10.399 51.721) (width 0.2) (layer "B.Cu") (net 5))
 (segment (start 10.399 62.49671) (end 12.07329 64.171) (width 0.2) (layer "B.Cu") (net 5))
 (segment (start 37.299 64.171) (end 38.88 62.59) (width 0.2) (layer "B.Cu") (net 5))
 (segment (start 10.399 51.721) (end 10.399 62.49671) (width 0.2) (layer "B.Cu") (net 5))
 (segment (start 12.07329 64.171) (end 37.299 64.171) (width 0.2) (layer "B.Cu") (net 5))
 (segment (start 37.391 85.051) (end 36.34 84) (width 0.2) (layer "B.Cu") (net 2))
 (segment (start 46.052 80.29076) (end 41.29176 85.051) (width 0.2) (layer "B.Cu") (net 2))
 (segment (start 38.9091 53.975) (end 46.052 61.1179) (width 0.2) (layer "B.Cu") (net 2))
 (segment (start 46.052 61.1179) (end 46.052 80.29076) (width 0.2) (layer "B.Cu") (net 2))
 (segment (start 36.105 53.975) (end 38.9091 53.975) (width 0.2) (layer "B.Cu") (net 2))
 (segment (start 41.29176 85.051) (end 37.391 85.051) (width 0.2) (layer "B.Cu") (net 2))
 (segment (start 26.897471 59.229) (end 38.88 71.211529) (width 0.2) (layer "F.Cu") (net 8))
 (segment (start 38.88 71.211529) (end 38.88 84) (width 0.2) (layer "F.Cu") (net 8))
 (segment (start 12.995 53.975) (end 18.249 59.229) (width 0.2) (layer "F.Cu") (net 8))
 (segment (start 18.249 59.229) (end 26.897471 59.229) (width 0.2) (layer "F.Cu") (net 8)))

